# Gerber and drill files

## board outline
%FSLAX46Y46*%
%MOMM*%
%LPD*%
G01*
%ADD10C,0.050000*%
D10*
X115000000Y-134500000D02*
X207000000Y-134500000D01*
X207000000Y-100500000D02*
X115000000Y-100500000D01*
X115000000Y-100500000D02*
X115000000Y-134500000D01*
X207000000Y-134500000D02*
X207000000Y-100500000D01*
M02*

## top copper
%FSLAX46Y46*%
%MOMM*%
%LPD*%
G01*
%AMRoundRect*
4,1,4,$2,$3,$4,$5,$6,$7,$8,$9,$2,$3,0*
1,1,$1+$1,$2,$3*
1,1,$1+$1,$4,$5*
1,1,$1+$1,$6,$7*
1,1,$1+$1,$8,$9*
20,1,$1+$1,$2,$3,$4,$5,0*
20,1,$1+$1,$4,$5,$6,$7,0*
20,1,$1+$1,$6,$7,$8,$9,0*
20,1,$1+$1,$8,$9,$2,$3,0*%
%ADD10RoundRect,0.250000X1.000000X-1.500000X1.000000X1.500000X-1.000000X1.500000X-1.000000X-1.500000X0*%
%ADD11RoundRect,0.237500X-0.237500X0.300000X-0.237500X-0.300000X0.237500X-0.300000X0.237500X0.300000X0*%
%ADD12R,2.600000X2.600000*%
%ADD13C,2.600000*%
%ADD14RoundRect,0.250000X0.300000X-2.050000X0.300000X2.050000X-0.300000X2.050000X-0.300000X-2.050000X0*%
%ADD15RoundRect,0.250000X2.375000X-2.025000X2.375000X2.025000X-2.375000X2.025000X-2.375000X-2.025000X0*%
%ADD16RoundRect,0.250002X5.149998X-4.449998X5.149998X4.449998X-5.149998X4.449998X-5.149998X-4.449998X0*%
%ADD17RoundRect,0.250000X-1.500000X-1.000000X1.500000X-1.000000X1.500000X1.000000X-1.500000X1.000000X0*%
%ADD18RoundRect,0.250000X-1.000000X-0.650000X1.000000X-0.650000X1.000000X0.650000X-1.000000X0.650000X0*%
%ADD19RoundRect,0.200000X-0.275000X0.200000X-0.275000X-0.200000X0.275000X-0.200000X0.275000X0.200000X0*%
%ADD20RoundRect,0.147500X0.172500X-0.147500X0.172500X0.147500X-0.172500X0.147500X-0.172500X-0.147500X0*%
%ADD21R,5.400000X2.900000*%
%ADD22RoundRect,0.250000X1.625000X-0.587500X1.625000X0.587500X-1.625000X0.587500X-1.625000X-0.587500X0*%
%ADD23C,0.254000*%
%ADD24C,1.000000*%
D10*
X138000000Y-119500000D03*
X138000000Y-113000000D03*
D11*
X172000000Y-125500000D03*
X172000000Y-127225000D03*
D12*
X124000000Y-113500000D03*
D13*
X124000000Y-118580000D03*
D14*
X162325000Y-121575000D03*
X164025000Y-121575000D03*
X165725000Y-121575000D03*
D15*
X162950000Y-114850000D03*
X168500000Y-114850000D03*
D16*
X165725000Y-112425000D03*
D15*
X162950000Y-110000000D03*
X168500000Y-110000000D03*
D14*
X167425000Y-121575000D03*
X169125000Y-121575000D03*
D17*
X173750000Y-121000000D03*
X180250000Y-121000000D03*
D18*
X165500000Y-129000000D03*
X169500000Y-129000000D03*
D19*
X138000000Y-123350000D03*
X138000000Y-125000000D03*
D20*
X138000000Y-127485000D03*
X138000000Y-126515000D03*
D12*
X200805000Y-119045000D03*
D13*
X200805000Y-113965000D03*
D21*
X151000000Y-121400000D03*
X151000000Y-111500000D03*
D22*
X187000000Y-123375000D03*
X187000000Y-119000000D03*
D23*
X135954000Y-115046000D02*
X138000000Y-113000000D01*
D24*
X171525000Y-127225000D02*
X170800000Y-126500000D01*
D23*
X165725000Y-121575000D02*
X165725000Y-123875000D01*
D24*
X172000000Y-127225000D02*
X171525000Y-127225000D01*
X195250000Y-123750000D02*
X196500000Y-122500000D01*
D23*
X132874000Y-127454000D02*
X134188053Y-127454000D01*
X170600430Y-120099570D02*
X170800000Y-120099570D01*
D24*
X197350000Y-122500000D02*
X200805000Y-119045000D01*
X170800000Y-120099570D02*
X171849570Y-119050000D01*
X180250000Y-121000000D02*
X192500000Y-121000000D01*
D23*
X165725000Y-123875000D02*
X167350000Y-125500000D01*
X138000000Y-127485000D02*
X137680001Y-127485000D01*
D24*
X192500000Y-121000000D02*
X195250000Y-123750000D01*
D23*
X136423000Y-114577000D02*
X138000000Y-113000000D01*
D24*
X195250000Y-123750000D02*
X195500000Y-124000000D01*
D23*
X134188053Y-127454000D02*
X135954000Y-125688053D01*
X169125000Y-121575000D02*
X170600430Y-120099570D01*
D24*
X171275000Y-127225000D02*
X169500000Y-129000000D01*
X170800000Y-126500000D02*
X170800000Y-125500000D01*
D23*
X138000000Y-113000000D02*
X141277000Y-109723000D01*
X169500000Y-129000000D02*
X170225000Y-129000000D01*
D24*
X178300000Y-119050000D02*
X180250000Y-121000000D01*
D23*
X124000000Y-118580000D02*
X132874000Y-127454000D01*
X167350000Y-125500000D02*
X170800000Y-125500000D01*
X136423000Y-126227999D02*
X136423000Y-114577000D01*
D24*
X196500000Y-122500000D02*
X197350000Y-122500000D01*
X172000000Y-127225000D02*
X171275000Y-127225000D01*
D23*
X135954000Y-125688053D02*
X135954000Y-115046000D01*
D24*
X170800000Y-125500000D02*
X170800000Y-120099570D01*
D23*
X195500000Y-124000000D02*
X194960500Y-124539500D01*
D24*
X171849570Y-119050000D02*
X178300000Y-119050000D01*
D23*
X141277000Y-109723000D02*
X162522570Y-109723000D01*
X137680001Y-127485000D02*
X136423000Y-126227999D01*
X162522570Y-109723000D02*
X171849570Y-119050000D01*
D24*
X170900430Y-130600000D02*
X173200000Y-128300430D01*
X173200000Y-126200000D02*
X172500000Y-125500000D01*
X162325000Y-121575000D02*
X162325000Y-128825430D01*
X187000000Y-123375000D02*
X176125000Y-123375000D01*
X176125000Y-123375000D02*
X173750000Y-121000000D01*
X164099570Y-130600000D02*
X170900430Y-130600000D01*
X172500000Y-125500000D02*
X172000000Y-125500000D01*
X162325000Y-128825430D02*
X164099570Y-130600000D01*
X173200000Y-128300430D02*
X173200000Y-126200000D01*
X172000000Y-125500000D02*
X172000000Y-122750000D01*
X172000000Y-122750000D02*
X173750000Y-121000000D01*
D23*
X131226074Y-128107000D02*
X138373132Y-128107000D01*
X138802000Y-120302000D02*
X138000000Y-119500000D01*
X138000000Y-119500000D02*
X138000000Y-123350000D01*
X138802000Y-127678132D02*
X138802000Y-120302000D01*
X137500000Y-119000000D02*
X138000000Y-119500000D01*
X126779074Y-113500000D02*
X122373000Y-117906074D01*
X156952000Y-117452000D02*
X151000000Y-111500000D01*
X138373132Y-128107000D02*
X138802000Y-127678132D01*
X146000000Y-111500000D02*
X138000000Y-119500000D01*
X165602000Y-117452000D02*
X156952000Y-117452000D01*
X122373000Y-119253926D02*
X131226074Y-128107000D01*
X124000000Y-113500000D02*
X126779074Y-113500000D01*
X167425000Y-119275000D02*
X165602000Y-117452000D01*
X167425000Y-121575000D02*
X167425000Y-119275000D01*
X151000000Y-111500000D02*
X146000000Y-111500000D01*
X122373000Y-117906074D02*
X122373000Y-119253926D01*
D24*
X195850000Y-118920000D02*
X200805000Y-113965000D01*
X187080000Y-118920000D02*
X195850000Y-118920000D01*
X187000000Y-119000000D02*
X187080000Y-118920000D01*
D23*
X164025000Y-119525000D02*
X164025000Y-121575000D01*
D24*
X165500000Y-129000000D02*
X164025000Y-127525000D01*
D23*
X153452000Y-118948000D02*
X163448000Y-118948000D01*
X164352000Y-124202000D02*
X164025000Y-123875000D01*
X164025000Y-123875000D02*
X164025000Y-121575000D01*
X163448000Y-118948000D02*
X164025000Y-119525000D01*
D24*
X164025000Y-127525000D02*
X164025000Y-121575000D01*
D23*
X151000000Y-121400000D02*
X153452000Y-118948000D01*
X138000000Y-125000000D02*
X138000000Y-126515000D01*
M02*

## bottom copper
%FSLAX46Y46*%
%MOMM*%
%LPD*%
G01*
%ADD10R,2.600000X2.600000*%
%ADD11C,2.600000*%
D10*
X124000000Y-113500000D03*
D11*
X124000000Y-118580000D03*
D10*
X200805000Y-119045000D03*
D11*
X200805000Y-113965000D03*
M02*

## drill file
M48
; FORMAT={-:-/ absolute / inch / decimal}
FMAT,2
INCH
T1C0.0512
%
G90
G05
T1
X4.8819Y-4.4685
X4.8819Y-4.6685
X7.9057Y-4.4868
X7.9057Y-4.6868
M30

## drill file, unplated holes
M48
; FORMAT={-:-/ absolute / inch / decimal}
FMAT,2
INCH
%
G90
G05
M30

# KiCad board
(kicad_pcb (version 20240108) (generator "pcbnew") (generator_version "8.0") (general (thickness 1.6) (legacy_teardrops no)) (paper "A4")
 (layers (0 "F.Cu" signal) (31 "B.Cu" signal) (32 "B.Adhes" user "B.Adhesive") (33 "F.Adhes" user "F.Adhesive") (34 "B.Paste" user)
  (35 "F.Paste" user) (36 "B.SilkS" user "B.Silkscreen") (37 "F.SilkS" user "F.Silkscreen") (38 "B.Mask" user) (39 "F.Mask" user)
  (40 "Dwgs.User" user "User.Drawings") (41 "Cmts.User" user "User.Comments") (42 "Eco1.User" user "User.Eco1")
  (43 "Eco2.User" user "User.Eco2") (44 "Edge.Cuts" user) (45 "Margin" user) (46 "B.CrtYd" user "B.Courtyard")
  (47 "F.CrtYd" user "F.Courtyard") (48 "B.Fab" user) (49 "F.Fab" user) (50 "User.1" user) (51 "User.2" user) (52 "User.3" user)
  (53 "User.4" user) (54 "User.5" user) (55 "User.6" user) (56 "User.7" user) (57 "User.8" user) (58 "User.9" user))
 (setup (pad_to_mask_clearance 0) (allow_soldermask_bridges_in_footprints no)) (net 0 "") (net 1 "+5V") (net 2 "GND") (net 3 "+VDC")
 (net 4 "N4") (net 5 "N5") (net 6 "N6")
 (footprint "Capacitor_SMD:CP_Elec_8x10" (layer "F.Cu") (at 138 116.25 90)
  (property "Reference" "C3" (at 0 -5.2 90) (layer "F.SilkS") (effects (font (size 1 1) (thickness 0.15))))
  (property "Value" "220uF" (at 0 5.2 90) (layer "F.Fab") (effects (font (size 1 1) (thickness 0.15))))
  (pad "1" smd roundrect (at -3.25 0 90) (size 3.5 2.5) (layers "F.Cu" "F.Paste" "F.Mask") (roundrect_rratio 0.1) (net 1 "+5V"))
  (pad "2" smd roundrect (at 3.25 0 90) (size 3.5 2.5) (layers "F.Cu" "F.Paste" "F.Mask") (roundrect_rratio 0.1) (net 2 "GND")))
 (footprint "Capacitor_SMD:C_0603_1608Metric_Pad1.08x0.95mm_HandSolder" (layer "F.Cu") (at 172 126.3625 -90)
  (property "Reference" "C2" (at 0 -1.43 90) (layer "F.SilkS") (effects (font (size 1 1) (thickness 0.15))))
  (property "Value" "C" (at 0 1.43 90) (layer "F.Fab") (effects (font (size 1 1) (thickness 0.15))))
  (pad "1" smd roundrect (at -0.8625 0 270) (size 1.075 0.95) (layers "F.Cu" "F.Paste" "F.Mask") (roundrect_rratio 0.25) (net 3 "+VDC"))
  (pad "2" smd roundrect (at 0.8625 0 270) (size 1.075 0.95) (layers "F.Cu" "F.Paste" "F.Mask") (roundrect_rratio 0.25) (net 2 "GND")))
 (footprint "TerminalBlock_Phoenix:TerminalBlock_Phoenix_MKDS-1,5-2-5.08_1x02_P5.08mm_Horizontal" (layer "F.Cu") (at 124 113.5 -90)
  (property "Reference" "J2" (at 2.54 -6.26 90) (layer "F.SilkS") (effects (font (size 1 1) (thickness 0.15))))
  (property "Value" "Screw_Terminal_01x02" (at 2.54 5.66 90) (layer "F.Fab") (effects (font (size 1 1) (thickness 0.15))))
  (pad "1" thru_hole rect (at 0 0 270) (size 2.6 2.6) (drill 1.3) (layers "*.Cu" "*.Mask") (remove_unused_layers no) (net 1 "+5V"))
  (pad "2" thru_hole circle (at 5.08 0 270) (size 2.6 2.6) (drill 1.3) (layers "*.Cu" "*.Mask") (remove_unused_layers no) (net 2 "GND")))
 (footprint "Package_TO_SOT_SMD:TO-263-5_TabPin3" (layer "F.Cu") (at 165.725 113.925 90)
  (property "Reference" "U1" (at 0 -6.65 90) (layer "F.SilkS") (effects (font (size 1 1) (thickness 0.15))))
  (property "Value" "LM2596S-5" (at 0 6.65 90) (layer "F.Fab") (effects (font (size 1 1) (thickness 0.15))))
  (pad "1" smd roundrect (at -7.65 -3.4 90) (size 4.6 1.1) (layers "F.Cu" "F.Paste" "F.Mask") (roundrect_rratio 0.227273) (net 3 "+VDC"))
  (pad "2" smd roundrect (at -7.65 -1.7 90) (size 4.6 1.1) (layers "F.Cu" "F.Paste" "F.Mask") (roundrect_rratio 0.227273) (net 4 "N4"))
  (pad "3" smd roundrect (at -7.65 0 90) (size 4.6 1.1) (layers "F.Cu" "F.Paste" "F.Mask") (roundrect_rratio 0.227273) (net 2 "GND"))
  (pad "3" smd roundrect (at -0.925 -2.775 90) (size 4.55 5.25) (layers "F.Cu" "F.Paste") (roundrect_rratio 0.054945) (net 2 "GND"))
  (pad "3" smd roundrect (at -0.925 2.775 90) (size 4.55 5.25) (layers "F.Cu" "F.Paste") (roundrect_rratio 0.054945) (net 2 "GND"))
  (pad "3" smd roundrect (at 1.5 0 90) (size 9.4 10.8) (layers "F.Cu" "F.Mask") (roundrect_rratio 0.026596) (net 2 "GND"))
  (pad "3" smd roundrect (at 3.925 -2.775 90) (size 4.55 5.25) (layers "F.Cu" "F.Paste") (roundrect_rratio 0.054945) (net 2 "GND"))
  (pad "3" smd roundrect (at 3.925 2.775 90) (size 4.55 5.25) (layers "F.Cu" "F.Paste") (roundrect_rratio 0.054945) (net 2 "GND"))
  (pad "4" smd roundrect (at -7.65 1.7 90) (size 4.6 1.1) (layers "F.Cu" "F.Paste" "F.Mask") (roundrect_rratio 0.227273) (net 1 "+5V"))
  (pad "5" smd roundrect (at -7.65 3.4 90) (size 4.6 1.1) (layers "F.Cu" "F.Paste" "F.Mask") (roundrect_rratio 0.227273) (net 2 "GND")))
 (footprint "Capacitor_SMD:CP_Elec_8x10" (layer "F.Cu") (at 177 121)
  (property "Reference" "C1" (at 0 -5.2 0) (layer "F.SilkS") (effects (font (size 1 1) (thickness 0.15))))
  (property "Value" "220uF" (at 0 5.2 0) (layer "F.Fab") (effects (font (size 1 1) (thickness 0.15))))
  (pad "1" smd roundrect (at -3.25 0) (size 3.5 2.5) (layers "F.Cu" "F.Paste" "F.Mask") (roundrect_rratio 0.1) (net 3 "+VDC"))
  (pad "2" smd roundrect (at 3.25 0) (size 3.5 2.5) (layers "F.Cu" "F.Paste" "F.Mask") (roundrect_rratio 0.1) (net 2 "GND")))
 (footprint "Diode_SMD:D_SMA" (layer "F.Cu") (at 167.5 129)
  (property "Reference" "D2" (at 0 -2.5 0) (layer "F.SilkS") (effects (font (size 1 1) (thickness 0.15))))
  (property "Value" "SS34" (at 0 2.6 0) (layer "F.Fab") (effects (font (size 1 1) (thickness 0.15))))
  (pad "1" smd roundrect (at -2 0) (size 2.5 1.8) (layers "F.Cu" "F.Paste" "F.Mask") (roundrect_rratio 0.1388888889) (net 4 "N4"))
  (pad "2" smd roundrect (at 2 0) (size 2.5 1.8) (layers "F.Cu" "F.Paste" "F.Mask") (roundrect_rratio 0.1388888889) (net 2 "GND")))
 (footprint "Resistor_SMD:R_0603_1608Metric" (layer "F.Cu") (at 138 124.175 -90)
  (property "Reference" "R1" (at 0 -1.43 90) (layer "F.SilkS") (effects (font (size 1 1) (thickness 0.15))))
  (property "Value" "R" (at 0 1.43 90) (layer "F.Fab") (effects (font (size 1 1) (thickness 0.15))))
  (pad "1" smd roundrect (at -0.825 0 270) (size 0.8 0.95) (layers "F.Cu" "F.Paste" "F.Mask") (roundrect_rratio 0.25) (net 1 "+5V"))
  (pad "2" smd roundrect (at 0.825 0 270) (size 0.8 0.95) (layers "F.Cu" "F.Paste" "F.Mask") (roundrect_rratio 0.25) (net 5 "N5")))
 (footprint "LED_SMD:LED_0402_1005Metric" (layer "F.Cu") (at 138 127 90)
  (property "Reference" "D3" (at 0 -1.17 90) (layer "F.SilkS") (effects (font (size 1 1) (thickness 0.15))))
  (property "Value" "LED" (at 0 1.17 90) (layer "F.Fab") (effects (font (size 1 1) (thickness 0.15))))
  (pad "1" smd roundrect (at -0.485 0 90) (size 0.59 0.64) (layers "F.Cu" "F.Paste" "F.Mask") (roundrect_rratio 0.25) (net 2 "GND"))
  (pad "2" smd roundrect (at 0.485 0 90) (size 0.59 0.64) (layers "F.Cu" "F.Paste" "F.Mask") (roundrect_rratio 0.25) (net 5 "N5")))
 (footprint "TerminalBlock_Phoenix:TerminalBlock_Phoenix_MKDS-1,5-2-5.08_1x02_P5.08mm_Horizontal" (layer "F.Cu") (at 200.805 119.045 90)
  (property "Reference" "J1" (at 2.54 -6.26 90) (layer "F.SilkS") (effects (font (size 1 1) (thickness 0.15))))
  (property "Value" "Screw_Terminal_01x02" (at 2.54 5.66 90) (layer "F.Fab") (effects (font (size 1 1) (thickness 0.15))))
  (pad "1" thru_hole rect (at 0 0 90) (size 2.6 2.6) (drill 1.3) (layers "*.Cu" "*.Mask") (remove_unused_layers no) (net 2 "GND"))
  (pad "2" thru_hole circle (at 5.08 0 90) (size 2.6 2.6) (drill 1.3) (layers "*.Cu" "*.Mask") (remove_unused_layers no) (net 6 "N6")))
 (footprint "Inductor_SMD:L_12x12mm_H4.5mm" (layer "F.Cu") (at 151 116.45 90)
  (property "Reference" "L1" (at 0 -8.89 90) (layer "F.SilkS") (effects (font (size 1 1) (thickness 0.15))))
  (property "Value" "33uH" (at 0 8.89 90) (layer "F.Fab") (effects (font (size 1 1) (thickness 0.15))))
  (pad "1" smd rect (at -4.95 0 90) (size 2.9 5.4) (layers "F.Cu" "F.Paste" "F.Mask") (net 4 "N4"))
  (pad "2" smd rect (at 4.95 0 90) (size 2.9 5.4) (layers "F.Cu" "F.Paste" "F.Mask") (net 1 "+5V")))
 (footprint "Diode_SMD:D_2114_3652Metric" (layer "F.Cu") (at 187 121.1875 90)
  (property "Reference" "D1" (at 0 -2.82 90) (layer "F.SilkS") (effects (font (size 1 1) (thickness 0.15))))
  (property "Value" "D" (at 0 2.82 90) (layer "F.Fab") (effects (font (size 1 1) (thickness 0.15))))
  (pad "1" smd roundrect (at -2.1875 0 90) (size 1.675 3.75) (layers "F.Cu" "F.Paste" "F.Mask") (roundrect_rratio 0.149254) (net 3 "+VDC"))
  (pad "2" smd roundrect (at 2.1875 0 90) (size 1.675 3.75) (layers "F.Cu" "F.Paste" "F.Mask") (roundrect_rratio 0.149254) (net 6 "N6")))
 (gr_line (start 115 134.5) (end 207 134.5) (stroke (width 0.05) (type default)) (layer "Edge.Cuts"))
 (gr_line (start 207 100.5) (end 115 100.5) (stroke (width 0.05) (type default)) (layer "Edge.Cuts"))
 (gr_line (start 115 100.5) (end 115 134.5) (stroke (width 0.05) (type default)) (layer "Edge.Cuts"))
 (gr_line (start 207 134.5) (end 207 100.5) (stroke (width 0.05) (type default)) (layer "Edge.Cuts"))
 (segment (start 135.954 115.046) (end 138 113) (width 0.254) (layer "F.Cu") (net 2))
 (segment (start 171.525 127.225) (end 170.8 126.5) (width 1) (layer "F.Cu") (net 2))
 (segment (start 165.725 121.575) (end 165.725 123.875) (width 0.254) (layer "F.Cu") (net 2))
 (segment (start 172 127.225) (end 171.525 127.225) (width 1) (layer "F.Cu") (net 2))
 (segment (start 195.25 123.75) (end 196.5 122.5) (width 1) (layer "F.Cu") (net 2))
 (segment (start 132.874 127.454) (end 134.188053 127.454) (width 0.254) (layer "F.Cu") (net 2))
 (segment (start 170.60043 120.09957) (end 170.8 120.09957) (width 0.254) (layer "F.Cu") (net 2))
 (segment (start 197.35 122.5) (end 200.805 119.045) (width 1) (layer "F.Cu") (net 2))
 (segment (start 170.8 120.09957) (end 171.84957 119.05) (width 1) (layer "F.Cu") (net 2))
 (segment (start 180.25 121) (end 192.5 121) (width 1) (layer "F.Cu") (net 2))
 (segment (start 165.725 123.875) (end 167.35 125.5) (width 0.254) (layer "F.Cu") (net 2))
 (segment (start 138 127.485) (end 137.680001 127.485) (width 0.254) (layer "F.Cu") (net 2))
 (segment (start 192.5 121) (end 195.25 123.75) (width 1) (layer "F.Cu") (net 2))
 (segment (start 136.423 114.577) (end 138 113) (width 0.254) (layer "F.Cu") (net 2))
 (segment (start 195.25 123.75) (end 195.5 124) (width 1) (layer "F.Cu") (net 2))
 (segment (start 134.188053 127.454) (end 135.954 125.688053) (width 0.254) (layer "F.Cu") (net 2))
 (segment (start 169.125 121.575) (end 170.60043 120.09957) (width 0.254) (layer "F.Cu") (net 2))
 (segment (start 171.275 127.225) (end 169.5 129) (width 1) (layer "F.Cu") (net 2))
 (segment (start 170.8 126.5) (end 170.8 125.5) (width 1) (layer "F.Cu") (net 2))
 (segment (start 138 113) (end 141.277 109.723) (width 0.254) (layer "F.Cu") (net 2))
 (segment (start 169.5 129) (end 170.225 129) (width 0.254) (layer "F.Cu") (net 2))
 (segment (start 178.3 119.05) (end 180.25 121) (width 1) (layer "F.Cu") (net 2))
 (segment (start 124 118.58) (end 132.874 127.454) (width 0.254) (layer "F.Cu") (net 2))
 (segment (start 167.35 125.5) (end 170.8 125.5) (width 0.254) (layer "F.Cu") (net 2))
 (segment (start 136.423 126.227999) (end 136.423 114.577) (width 0.254) (layer "F.Cu") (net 2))
 (segment (start 196.5 122.5) (end 197.35 122.5) (width 1) (layer "F.Cu") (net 2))
 (segment (start 172 127.225) (end 171.275 127.225) (width 1) (layer "F.Cu") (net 2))
 (segment (start 135.954 125.688053) (end 135.954 115.046) (width 0.254) (layer "F.Cu") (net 2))
 (segment (start 170.8 125.5) (end 170.8 120.09957) (width 1) (layer "F.Cu") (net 2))
 (segment (start 195.5 124) (end 194.9605 124.5395) (width 0.254) (layer "F.Cu") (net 2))
 (segment (start 171.84957 119.05) (end 178.3 119.05) (width 1) (layer "F.Cu") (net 2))
 (segment (start 141.277 109.723) (end 162.52257 109.723) (width 0.254) (layer "F.Cu") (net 2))
 (segment (start 137.680001 127.485) (end 136.423 126.227999) (width 0.254) (layer "F.Cu") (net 2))
 (segment (start 162.52257 109.723) (end 171.84957 119.05) (width 0.254) (layer "F.Cu") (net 2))
 (segment (start 170.90043 130.6) (end 173.2 128.30043) (width 1) (layer "F.Cu") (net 3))
 (segment (start 173.2 126.2) (end 172.5 125.5) (width 1) (layer "F.Cu") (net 3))
 (segment (start 162.325 121.575) (end 162.325 128.82543) (width 1) (layer "F.Cu") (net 3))
 (segment (start 187 123.375) (end 176.125 123.375) (width 1) (layer "F.Cu") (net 3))
 (segment (start 176.125 123.375) (end 173.75 121) (width 1) (layer "F.Cu") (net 3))
 (segment (start 164.09957 130.6) (end 170.90043 130.6) (width 1) (layer "F.Cu") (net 3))
 (segment (start 172.5 125.5) (end 172 125.5) (width 1) (layer "F.Cu") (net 3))
 (segment (start 162.325 128.82543) (end 164.09957 130.6) (width 1) (layer "F.Cu") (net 3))
 (segment (start 173.2 128.30043) (end 173.2 126.2) (width 1) (layer "F.Cu") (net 3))
 (segment (start 172 125.5) (end 172 122.75) (width 1) (layer "F.Cu") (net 3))
 (segment (start 172 122.75) (end 173.75 121) (width 1) (layer "F.Cu") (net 3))
 (segment (start 131.226074 128.107) (end 138.373132 128.107) (width 0.254) (layer "F.Cu") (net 1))
 (segment (start 138.802 120.302) (end 138 119.5) (width 0.254) (layer "F.Cu") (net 1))
 (segment (start 138 119.5) (end 138 123.35) (width 0.254) (layer "F.Cu") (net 1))
 (segment (start 138.802 127.678132) (end 138.802 120.302) (width 0.254) (layer "F.Cu") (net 1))
 (segment (start 137.5 119) (end 138 119.5) (width 0.254) (layer "F.Cu") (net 1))
 (segment (start 126.779074 113.5) (end 122.373 117.906074) (width 0.254) (layer "F.Cu") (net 1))
 (segment (start 156.952 117.452) (end 151 111.5) (width 0.254) (layer "F.Cu") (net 1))
 (segment (start 138.373132 128.107) (end 138.802 127.678132) (width 0.254) (layer "F.Cu") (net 1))
 (segment (start 146 111.5) (end 138 119.5) (width 0.254) (layer "F.Cu") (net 1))
 (segment (start 165.602 117.452) (end 156.952 117.452) (width 0.254) (layer "F.Cu") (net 1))
 (segment (start 122.373 119.253926) (end 131.226074 128.107) (width 0.254) (layer "F.Cu") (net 1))
 (segment (start 124 113.5) (end 126.779074 113.5) (width 0.254) (layer "F.Cu") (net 1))
 (segment (start 167.425 119.275) (end 165.602 117.452) (width 0.254) (layer "F.Cu") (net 1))
 (segment (start 167.425 121.575) (end 167.425 119.275) (width 0.254) (layer "F.Cu") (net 1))
 (segment (start 151 111.5) (end 146 111.5) (width 0.254) (layer "F.Cu") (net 1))
 (segment (start 122.373 117.906074) (end 122.373 119.253926) (width 0.254) (layer "F.Cu") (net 1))
 (segment (start 195.85 118.92) (end 200.805 113.965) (width 1) (layer "F.Cu") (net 6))
 (segment (start 187.08 118.92) (end 195.85 118.92) (width 1) (layer "F.Cu") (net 6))
 (segment (start 187 119) (end 187.08 118.92) (width 1) (layer "F.Cu") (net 6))
 (segment (start 164.025 119.525) (end 164.025 121.575) (width 0.254) (layer "F.Cu") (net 4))
 (segment (start 165.5 129) (end 164.025 127.525) (width 1) (layer "F.Cu") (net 4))
 (segment (start 153.452 118.948) (end 163.448 118.948) (width 0.254) (layer "F.Cu") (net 4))
 (segment (start 164.352 124.202) (end 164.025 123.875) (width 0.254) (layer "F.Cu") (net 4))
 (segment (start 164.025 123.875) (end 164.025 121.575) (width 0.254) (layer "F.Cu") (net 4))
 (segment (start 163.448 118.948) (end 164.025 119.525) (width 0.254) (layer "F.Cu") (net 4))
 (segment (start 164.025 127.525) (end 164.025 121.575) (width 1) (layer "F.Cu") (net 4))
 (segment (start 151 121.4) (end 153.452 118.948) (width 0.254) (layer "F.Cu") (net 4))
 (segment (start 138 125) (end 138 126.515) (width 0.254) (layer "F.Cu") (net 5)))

